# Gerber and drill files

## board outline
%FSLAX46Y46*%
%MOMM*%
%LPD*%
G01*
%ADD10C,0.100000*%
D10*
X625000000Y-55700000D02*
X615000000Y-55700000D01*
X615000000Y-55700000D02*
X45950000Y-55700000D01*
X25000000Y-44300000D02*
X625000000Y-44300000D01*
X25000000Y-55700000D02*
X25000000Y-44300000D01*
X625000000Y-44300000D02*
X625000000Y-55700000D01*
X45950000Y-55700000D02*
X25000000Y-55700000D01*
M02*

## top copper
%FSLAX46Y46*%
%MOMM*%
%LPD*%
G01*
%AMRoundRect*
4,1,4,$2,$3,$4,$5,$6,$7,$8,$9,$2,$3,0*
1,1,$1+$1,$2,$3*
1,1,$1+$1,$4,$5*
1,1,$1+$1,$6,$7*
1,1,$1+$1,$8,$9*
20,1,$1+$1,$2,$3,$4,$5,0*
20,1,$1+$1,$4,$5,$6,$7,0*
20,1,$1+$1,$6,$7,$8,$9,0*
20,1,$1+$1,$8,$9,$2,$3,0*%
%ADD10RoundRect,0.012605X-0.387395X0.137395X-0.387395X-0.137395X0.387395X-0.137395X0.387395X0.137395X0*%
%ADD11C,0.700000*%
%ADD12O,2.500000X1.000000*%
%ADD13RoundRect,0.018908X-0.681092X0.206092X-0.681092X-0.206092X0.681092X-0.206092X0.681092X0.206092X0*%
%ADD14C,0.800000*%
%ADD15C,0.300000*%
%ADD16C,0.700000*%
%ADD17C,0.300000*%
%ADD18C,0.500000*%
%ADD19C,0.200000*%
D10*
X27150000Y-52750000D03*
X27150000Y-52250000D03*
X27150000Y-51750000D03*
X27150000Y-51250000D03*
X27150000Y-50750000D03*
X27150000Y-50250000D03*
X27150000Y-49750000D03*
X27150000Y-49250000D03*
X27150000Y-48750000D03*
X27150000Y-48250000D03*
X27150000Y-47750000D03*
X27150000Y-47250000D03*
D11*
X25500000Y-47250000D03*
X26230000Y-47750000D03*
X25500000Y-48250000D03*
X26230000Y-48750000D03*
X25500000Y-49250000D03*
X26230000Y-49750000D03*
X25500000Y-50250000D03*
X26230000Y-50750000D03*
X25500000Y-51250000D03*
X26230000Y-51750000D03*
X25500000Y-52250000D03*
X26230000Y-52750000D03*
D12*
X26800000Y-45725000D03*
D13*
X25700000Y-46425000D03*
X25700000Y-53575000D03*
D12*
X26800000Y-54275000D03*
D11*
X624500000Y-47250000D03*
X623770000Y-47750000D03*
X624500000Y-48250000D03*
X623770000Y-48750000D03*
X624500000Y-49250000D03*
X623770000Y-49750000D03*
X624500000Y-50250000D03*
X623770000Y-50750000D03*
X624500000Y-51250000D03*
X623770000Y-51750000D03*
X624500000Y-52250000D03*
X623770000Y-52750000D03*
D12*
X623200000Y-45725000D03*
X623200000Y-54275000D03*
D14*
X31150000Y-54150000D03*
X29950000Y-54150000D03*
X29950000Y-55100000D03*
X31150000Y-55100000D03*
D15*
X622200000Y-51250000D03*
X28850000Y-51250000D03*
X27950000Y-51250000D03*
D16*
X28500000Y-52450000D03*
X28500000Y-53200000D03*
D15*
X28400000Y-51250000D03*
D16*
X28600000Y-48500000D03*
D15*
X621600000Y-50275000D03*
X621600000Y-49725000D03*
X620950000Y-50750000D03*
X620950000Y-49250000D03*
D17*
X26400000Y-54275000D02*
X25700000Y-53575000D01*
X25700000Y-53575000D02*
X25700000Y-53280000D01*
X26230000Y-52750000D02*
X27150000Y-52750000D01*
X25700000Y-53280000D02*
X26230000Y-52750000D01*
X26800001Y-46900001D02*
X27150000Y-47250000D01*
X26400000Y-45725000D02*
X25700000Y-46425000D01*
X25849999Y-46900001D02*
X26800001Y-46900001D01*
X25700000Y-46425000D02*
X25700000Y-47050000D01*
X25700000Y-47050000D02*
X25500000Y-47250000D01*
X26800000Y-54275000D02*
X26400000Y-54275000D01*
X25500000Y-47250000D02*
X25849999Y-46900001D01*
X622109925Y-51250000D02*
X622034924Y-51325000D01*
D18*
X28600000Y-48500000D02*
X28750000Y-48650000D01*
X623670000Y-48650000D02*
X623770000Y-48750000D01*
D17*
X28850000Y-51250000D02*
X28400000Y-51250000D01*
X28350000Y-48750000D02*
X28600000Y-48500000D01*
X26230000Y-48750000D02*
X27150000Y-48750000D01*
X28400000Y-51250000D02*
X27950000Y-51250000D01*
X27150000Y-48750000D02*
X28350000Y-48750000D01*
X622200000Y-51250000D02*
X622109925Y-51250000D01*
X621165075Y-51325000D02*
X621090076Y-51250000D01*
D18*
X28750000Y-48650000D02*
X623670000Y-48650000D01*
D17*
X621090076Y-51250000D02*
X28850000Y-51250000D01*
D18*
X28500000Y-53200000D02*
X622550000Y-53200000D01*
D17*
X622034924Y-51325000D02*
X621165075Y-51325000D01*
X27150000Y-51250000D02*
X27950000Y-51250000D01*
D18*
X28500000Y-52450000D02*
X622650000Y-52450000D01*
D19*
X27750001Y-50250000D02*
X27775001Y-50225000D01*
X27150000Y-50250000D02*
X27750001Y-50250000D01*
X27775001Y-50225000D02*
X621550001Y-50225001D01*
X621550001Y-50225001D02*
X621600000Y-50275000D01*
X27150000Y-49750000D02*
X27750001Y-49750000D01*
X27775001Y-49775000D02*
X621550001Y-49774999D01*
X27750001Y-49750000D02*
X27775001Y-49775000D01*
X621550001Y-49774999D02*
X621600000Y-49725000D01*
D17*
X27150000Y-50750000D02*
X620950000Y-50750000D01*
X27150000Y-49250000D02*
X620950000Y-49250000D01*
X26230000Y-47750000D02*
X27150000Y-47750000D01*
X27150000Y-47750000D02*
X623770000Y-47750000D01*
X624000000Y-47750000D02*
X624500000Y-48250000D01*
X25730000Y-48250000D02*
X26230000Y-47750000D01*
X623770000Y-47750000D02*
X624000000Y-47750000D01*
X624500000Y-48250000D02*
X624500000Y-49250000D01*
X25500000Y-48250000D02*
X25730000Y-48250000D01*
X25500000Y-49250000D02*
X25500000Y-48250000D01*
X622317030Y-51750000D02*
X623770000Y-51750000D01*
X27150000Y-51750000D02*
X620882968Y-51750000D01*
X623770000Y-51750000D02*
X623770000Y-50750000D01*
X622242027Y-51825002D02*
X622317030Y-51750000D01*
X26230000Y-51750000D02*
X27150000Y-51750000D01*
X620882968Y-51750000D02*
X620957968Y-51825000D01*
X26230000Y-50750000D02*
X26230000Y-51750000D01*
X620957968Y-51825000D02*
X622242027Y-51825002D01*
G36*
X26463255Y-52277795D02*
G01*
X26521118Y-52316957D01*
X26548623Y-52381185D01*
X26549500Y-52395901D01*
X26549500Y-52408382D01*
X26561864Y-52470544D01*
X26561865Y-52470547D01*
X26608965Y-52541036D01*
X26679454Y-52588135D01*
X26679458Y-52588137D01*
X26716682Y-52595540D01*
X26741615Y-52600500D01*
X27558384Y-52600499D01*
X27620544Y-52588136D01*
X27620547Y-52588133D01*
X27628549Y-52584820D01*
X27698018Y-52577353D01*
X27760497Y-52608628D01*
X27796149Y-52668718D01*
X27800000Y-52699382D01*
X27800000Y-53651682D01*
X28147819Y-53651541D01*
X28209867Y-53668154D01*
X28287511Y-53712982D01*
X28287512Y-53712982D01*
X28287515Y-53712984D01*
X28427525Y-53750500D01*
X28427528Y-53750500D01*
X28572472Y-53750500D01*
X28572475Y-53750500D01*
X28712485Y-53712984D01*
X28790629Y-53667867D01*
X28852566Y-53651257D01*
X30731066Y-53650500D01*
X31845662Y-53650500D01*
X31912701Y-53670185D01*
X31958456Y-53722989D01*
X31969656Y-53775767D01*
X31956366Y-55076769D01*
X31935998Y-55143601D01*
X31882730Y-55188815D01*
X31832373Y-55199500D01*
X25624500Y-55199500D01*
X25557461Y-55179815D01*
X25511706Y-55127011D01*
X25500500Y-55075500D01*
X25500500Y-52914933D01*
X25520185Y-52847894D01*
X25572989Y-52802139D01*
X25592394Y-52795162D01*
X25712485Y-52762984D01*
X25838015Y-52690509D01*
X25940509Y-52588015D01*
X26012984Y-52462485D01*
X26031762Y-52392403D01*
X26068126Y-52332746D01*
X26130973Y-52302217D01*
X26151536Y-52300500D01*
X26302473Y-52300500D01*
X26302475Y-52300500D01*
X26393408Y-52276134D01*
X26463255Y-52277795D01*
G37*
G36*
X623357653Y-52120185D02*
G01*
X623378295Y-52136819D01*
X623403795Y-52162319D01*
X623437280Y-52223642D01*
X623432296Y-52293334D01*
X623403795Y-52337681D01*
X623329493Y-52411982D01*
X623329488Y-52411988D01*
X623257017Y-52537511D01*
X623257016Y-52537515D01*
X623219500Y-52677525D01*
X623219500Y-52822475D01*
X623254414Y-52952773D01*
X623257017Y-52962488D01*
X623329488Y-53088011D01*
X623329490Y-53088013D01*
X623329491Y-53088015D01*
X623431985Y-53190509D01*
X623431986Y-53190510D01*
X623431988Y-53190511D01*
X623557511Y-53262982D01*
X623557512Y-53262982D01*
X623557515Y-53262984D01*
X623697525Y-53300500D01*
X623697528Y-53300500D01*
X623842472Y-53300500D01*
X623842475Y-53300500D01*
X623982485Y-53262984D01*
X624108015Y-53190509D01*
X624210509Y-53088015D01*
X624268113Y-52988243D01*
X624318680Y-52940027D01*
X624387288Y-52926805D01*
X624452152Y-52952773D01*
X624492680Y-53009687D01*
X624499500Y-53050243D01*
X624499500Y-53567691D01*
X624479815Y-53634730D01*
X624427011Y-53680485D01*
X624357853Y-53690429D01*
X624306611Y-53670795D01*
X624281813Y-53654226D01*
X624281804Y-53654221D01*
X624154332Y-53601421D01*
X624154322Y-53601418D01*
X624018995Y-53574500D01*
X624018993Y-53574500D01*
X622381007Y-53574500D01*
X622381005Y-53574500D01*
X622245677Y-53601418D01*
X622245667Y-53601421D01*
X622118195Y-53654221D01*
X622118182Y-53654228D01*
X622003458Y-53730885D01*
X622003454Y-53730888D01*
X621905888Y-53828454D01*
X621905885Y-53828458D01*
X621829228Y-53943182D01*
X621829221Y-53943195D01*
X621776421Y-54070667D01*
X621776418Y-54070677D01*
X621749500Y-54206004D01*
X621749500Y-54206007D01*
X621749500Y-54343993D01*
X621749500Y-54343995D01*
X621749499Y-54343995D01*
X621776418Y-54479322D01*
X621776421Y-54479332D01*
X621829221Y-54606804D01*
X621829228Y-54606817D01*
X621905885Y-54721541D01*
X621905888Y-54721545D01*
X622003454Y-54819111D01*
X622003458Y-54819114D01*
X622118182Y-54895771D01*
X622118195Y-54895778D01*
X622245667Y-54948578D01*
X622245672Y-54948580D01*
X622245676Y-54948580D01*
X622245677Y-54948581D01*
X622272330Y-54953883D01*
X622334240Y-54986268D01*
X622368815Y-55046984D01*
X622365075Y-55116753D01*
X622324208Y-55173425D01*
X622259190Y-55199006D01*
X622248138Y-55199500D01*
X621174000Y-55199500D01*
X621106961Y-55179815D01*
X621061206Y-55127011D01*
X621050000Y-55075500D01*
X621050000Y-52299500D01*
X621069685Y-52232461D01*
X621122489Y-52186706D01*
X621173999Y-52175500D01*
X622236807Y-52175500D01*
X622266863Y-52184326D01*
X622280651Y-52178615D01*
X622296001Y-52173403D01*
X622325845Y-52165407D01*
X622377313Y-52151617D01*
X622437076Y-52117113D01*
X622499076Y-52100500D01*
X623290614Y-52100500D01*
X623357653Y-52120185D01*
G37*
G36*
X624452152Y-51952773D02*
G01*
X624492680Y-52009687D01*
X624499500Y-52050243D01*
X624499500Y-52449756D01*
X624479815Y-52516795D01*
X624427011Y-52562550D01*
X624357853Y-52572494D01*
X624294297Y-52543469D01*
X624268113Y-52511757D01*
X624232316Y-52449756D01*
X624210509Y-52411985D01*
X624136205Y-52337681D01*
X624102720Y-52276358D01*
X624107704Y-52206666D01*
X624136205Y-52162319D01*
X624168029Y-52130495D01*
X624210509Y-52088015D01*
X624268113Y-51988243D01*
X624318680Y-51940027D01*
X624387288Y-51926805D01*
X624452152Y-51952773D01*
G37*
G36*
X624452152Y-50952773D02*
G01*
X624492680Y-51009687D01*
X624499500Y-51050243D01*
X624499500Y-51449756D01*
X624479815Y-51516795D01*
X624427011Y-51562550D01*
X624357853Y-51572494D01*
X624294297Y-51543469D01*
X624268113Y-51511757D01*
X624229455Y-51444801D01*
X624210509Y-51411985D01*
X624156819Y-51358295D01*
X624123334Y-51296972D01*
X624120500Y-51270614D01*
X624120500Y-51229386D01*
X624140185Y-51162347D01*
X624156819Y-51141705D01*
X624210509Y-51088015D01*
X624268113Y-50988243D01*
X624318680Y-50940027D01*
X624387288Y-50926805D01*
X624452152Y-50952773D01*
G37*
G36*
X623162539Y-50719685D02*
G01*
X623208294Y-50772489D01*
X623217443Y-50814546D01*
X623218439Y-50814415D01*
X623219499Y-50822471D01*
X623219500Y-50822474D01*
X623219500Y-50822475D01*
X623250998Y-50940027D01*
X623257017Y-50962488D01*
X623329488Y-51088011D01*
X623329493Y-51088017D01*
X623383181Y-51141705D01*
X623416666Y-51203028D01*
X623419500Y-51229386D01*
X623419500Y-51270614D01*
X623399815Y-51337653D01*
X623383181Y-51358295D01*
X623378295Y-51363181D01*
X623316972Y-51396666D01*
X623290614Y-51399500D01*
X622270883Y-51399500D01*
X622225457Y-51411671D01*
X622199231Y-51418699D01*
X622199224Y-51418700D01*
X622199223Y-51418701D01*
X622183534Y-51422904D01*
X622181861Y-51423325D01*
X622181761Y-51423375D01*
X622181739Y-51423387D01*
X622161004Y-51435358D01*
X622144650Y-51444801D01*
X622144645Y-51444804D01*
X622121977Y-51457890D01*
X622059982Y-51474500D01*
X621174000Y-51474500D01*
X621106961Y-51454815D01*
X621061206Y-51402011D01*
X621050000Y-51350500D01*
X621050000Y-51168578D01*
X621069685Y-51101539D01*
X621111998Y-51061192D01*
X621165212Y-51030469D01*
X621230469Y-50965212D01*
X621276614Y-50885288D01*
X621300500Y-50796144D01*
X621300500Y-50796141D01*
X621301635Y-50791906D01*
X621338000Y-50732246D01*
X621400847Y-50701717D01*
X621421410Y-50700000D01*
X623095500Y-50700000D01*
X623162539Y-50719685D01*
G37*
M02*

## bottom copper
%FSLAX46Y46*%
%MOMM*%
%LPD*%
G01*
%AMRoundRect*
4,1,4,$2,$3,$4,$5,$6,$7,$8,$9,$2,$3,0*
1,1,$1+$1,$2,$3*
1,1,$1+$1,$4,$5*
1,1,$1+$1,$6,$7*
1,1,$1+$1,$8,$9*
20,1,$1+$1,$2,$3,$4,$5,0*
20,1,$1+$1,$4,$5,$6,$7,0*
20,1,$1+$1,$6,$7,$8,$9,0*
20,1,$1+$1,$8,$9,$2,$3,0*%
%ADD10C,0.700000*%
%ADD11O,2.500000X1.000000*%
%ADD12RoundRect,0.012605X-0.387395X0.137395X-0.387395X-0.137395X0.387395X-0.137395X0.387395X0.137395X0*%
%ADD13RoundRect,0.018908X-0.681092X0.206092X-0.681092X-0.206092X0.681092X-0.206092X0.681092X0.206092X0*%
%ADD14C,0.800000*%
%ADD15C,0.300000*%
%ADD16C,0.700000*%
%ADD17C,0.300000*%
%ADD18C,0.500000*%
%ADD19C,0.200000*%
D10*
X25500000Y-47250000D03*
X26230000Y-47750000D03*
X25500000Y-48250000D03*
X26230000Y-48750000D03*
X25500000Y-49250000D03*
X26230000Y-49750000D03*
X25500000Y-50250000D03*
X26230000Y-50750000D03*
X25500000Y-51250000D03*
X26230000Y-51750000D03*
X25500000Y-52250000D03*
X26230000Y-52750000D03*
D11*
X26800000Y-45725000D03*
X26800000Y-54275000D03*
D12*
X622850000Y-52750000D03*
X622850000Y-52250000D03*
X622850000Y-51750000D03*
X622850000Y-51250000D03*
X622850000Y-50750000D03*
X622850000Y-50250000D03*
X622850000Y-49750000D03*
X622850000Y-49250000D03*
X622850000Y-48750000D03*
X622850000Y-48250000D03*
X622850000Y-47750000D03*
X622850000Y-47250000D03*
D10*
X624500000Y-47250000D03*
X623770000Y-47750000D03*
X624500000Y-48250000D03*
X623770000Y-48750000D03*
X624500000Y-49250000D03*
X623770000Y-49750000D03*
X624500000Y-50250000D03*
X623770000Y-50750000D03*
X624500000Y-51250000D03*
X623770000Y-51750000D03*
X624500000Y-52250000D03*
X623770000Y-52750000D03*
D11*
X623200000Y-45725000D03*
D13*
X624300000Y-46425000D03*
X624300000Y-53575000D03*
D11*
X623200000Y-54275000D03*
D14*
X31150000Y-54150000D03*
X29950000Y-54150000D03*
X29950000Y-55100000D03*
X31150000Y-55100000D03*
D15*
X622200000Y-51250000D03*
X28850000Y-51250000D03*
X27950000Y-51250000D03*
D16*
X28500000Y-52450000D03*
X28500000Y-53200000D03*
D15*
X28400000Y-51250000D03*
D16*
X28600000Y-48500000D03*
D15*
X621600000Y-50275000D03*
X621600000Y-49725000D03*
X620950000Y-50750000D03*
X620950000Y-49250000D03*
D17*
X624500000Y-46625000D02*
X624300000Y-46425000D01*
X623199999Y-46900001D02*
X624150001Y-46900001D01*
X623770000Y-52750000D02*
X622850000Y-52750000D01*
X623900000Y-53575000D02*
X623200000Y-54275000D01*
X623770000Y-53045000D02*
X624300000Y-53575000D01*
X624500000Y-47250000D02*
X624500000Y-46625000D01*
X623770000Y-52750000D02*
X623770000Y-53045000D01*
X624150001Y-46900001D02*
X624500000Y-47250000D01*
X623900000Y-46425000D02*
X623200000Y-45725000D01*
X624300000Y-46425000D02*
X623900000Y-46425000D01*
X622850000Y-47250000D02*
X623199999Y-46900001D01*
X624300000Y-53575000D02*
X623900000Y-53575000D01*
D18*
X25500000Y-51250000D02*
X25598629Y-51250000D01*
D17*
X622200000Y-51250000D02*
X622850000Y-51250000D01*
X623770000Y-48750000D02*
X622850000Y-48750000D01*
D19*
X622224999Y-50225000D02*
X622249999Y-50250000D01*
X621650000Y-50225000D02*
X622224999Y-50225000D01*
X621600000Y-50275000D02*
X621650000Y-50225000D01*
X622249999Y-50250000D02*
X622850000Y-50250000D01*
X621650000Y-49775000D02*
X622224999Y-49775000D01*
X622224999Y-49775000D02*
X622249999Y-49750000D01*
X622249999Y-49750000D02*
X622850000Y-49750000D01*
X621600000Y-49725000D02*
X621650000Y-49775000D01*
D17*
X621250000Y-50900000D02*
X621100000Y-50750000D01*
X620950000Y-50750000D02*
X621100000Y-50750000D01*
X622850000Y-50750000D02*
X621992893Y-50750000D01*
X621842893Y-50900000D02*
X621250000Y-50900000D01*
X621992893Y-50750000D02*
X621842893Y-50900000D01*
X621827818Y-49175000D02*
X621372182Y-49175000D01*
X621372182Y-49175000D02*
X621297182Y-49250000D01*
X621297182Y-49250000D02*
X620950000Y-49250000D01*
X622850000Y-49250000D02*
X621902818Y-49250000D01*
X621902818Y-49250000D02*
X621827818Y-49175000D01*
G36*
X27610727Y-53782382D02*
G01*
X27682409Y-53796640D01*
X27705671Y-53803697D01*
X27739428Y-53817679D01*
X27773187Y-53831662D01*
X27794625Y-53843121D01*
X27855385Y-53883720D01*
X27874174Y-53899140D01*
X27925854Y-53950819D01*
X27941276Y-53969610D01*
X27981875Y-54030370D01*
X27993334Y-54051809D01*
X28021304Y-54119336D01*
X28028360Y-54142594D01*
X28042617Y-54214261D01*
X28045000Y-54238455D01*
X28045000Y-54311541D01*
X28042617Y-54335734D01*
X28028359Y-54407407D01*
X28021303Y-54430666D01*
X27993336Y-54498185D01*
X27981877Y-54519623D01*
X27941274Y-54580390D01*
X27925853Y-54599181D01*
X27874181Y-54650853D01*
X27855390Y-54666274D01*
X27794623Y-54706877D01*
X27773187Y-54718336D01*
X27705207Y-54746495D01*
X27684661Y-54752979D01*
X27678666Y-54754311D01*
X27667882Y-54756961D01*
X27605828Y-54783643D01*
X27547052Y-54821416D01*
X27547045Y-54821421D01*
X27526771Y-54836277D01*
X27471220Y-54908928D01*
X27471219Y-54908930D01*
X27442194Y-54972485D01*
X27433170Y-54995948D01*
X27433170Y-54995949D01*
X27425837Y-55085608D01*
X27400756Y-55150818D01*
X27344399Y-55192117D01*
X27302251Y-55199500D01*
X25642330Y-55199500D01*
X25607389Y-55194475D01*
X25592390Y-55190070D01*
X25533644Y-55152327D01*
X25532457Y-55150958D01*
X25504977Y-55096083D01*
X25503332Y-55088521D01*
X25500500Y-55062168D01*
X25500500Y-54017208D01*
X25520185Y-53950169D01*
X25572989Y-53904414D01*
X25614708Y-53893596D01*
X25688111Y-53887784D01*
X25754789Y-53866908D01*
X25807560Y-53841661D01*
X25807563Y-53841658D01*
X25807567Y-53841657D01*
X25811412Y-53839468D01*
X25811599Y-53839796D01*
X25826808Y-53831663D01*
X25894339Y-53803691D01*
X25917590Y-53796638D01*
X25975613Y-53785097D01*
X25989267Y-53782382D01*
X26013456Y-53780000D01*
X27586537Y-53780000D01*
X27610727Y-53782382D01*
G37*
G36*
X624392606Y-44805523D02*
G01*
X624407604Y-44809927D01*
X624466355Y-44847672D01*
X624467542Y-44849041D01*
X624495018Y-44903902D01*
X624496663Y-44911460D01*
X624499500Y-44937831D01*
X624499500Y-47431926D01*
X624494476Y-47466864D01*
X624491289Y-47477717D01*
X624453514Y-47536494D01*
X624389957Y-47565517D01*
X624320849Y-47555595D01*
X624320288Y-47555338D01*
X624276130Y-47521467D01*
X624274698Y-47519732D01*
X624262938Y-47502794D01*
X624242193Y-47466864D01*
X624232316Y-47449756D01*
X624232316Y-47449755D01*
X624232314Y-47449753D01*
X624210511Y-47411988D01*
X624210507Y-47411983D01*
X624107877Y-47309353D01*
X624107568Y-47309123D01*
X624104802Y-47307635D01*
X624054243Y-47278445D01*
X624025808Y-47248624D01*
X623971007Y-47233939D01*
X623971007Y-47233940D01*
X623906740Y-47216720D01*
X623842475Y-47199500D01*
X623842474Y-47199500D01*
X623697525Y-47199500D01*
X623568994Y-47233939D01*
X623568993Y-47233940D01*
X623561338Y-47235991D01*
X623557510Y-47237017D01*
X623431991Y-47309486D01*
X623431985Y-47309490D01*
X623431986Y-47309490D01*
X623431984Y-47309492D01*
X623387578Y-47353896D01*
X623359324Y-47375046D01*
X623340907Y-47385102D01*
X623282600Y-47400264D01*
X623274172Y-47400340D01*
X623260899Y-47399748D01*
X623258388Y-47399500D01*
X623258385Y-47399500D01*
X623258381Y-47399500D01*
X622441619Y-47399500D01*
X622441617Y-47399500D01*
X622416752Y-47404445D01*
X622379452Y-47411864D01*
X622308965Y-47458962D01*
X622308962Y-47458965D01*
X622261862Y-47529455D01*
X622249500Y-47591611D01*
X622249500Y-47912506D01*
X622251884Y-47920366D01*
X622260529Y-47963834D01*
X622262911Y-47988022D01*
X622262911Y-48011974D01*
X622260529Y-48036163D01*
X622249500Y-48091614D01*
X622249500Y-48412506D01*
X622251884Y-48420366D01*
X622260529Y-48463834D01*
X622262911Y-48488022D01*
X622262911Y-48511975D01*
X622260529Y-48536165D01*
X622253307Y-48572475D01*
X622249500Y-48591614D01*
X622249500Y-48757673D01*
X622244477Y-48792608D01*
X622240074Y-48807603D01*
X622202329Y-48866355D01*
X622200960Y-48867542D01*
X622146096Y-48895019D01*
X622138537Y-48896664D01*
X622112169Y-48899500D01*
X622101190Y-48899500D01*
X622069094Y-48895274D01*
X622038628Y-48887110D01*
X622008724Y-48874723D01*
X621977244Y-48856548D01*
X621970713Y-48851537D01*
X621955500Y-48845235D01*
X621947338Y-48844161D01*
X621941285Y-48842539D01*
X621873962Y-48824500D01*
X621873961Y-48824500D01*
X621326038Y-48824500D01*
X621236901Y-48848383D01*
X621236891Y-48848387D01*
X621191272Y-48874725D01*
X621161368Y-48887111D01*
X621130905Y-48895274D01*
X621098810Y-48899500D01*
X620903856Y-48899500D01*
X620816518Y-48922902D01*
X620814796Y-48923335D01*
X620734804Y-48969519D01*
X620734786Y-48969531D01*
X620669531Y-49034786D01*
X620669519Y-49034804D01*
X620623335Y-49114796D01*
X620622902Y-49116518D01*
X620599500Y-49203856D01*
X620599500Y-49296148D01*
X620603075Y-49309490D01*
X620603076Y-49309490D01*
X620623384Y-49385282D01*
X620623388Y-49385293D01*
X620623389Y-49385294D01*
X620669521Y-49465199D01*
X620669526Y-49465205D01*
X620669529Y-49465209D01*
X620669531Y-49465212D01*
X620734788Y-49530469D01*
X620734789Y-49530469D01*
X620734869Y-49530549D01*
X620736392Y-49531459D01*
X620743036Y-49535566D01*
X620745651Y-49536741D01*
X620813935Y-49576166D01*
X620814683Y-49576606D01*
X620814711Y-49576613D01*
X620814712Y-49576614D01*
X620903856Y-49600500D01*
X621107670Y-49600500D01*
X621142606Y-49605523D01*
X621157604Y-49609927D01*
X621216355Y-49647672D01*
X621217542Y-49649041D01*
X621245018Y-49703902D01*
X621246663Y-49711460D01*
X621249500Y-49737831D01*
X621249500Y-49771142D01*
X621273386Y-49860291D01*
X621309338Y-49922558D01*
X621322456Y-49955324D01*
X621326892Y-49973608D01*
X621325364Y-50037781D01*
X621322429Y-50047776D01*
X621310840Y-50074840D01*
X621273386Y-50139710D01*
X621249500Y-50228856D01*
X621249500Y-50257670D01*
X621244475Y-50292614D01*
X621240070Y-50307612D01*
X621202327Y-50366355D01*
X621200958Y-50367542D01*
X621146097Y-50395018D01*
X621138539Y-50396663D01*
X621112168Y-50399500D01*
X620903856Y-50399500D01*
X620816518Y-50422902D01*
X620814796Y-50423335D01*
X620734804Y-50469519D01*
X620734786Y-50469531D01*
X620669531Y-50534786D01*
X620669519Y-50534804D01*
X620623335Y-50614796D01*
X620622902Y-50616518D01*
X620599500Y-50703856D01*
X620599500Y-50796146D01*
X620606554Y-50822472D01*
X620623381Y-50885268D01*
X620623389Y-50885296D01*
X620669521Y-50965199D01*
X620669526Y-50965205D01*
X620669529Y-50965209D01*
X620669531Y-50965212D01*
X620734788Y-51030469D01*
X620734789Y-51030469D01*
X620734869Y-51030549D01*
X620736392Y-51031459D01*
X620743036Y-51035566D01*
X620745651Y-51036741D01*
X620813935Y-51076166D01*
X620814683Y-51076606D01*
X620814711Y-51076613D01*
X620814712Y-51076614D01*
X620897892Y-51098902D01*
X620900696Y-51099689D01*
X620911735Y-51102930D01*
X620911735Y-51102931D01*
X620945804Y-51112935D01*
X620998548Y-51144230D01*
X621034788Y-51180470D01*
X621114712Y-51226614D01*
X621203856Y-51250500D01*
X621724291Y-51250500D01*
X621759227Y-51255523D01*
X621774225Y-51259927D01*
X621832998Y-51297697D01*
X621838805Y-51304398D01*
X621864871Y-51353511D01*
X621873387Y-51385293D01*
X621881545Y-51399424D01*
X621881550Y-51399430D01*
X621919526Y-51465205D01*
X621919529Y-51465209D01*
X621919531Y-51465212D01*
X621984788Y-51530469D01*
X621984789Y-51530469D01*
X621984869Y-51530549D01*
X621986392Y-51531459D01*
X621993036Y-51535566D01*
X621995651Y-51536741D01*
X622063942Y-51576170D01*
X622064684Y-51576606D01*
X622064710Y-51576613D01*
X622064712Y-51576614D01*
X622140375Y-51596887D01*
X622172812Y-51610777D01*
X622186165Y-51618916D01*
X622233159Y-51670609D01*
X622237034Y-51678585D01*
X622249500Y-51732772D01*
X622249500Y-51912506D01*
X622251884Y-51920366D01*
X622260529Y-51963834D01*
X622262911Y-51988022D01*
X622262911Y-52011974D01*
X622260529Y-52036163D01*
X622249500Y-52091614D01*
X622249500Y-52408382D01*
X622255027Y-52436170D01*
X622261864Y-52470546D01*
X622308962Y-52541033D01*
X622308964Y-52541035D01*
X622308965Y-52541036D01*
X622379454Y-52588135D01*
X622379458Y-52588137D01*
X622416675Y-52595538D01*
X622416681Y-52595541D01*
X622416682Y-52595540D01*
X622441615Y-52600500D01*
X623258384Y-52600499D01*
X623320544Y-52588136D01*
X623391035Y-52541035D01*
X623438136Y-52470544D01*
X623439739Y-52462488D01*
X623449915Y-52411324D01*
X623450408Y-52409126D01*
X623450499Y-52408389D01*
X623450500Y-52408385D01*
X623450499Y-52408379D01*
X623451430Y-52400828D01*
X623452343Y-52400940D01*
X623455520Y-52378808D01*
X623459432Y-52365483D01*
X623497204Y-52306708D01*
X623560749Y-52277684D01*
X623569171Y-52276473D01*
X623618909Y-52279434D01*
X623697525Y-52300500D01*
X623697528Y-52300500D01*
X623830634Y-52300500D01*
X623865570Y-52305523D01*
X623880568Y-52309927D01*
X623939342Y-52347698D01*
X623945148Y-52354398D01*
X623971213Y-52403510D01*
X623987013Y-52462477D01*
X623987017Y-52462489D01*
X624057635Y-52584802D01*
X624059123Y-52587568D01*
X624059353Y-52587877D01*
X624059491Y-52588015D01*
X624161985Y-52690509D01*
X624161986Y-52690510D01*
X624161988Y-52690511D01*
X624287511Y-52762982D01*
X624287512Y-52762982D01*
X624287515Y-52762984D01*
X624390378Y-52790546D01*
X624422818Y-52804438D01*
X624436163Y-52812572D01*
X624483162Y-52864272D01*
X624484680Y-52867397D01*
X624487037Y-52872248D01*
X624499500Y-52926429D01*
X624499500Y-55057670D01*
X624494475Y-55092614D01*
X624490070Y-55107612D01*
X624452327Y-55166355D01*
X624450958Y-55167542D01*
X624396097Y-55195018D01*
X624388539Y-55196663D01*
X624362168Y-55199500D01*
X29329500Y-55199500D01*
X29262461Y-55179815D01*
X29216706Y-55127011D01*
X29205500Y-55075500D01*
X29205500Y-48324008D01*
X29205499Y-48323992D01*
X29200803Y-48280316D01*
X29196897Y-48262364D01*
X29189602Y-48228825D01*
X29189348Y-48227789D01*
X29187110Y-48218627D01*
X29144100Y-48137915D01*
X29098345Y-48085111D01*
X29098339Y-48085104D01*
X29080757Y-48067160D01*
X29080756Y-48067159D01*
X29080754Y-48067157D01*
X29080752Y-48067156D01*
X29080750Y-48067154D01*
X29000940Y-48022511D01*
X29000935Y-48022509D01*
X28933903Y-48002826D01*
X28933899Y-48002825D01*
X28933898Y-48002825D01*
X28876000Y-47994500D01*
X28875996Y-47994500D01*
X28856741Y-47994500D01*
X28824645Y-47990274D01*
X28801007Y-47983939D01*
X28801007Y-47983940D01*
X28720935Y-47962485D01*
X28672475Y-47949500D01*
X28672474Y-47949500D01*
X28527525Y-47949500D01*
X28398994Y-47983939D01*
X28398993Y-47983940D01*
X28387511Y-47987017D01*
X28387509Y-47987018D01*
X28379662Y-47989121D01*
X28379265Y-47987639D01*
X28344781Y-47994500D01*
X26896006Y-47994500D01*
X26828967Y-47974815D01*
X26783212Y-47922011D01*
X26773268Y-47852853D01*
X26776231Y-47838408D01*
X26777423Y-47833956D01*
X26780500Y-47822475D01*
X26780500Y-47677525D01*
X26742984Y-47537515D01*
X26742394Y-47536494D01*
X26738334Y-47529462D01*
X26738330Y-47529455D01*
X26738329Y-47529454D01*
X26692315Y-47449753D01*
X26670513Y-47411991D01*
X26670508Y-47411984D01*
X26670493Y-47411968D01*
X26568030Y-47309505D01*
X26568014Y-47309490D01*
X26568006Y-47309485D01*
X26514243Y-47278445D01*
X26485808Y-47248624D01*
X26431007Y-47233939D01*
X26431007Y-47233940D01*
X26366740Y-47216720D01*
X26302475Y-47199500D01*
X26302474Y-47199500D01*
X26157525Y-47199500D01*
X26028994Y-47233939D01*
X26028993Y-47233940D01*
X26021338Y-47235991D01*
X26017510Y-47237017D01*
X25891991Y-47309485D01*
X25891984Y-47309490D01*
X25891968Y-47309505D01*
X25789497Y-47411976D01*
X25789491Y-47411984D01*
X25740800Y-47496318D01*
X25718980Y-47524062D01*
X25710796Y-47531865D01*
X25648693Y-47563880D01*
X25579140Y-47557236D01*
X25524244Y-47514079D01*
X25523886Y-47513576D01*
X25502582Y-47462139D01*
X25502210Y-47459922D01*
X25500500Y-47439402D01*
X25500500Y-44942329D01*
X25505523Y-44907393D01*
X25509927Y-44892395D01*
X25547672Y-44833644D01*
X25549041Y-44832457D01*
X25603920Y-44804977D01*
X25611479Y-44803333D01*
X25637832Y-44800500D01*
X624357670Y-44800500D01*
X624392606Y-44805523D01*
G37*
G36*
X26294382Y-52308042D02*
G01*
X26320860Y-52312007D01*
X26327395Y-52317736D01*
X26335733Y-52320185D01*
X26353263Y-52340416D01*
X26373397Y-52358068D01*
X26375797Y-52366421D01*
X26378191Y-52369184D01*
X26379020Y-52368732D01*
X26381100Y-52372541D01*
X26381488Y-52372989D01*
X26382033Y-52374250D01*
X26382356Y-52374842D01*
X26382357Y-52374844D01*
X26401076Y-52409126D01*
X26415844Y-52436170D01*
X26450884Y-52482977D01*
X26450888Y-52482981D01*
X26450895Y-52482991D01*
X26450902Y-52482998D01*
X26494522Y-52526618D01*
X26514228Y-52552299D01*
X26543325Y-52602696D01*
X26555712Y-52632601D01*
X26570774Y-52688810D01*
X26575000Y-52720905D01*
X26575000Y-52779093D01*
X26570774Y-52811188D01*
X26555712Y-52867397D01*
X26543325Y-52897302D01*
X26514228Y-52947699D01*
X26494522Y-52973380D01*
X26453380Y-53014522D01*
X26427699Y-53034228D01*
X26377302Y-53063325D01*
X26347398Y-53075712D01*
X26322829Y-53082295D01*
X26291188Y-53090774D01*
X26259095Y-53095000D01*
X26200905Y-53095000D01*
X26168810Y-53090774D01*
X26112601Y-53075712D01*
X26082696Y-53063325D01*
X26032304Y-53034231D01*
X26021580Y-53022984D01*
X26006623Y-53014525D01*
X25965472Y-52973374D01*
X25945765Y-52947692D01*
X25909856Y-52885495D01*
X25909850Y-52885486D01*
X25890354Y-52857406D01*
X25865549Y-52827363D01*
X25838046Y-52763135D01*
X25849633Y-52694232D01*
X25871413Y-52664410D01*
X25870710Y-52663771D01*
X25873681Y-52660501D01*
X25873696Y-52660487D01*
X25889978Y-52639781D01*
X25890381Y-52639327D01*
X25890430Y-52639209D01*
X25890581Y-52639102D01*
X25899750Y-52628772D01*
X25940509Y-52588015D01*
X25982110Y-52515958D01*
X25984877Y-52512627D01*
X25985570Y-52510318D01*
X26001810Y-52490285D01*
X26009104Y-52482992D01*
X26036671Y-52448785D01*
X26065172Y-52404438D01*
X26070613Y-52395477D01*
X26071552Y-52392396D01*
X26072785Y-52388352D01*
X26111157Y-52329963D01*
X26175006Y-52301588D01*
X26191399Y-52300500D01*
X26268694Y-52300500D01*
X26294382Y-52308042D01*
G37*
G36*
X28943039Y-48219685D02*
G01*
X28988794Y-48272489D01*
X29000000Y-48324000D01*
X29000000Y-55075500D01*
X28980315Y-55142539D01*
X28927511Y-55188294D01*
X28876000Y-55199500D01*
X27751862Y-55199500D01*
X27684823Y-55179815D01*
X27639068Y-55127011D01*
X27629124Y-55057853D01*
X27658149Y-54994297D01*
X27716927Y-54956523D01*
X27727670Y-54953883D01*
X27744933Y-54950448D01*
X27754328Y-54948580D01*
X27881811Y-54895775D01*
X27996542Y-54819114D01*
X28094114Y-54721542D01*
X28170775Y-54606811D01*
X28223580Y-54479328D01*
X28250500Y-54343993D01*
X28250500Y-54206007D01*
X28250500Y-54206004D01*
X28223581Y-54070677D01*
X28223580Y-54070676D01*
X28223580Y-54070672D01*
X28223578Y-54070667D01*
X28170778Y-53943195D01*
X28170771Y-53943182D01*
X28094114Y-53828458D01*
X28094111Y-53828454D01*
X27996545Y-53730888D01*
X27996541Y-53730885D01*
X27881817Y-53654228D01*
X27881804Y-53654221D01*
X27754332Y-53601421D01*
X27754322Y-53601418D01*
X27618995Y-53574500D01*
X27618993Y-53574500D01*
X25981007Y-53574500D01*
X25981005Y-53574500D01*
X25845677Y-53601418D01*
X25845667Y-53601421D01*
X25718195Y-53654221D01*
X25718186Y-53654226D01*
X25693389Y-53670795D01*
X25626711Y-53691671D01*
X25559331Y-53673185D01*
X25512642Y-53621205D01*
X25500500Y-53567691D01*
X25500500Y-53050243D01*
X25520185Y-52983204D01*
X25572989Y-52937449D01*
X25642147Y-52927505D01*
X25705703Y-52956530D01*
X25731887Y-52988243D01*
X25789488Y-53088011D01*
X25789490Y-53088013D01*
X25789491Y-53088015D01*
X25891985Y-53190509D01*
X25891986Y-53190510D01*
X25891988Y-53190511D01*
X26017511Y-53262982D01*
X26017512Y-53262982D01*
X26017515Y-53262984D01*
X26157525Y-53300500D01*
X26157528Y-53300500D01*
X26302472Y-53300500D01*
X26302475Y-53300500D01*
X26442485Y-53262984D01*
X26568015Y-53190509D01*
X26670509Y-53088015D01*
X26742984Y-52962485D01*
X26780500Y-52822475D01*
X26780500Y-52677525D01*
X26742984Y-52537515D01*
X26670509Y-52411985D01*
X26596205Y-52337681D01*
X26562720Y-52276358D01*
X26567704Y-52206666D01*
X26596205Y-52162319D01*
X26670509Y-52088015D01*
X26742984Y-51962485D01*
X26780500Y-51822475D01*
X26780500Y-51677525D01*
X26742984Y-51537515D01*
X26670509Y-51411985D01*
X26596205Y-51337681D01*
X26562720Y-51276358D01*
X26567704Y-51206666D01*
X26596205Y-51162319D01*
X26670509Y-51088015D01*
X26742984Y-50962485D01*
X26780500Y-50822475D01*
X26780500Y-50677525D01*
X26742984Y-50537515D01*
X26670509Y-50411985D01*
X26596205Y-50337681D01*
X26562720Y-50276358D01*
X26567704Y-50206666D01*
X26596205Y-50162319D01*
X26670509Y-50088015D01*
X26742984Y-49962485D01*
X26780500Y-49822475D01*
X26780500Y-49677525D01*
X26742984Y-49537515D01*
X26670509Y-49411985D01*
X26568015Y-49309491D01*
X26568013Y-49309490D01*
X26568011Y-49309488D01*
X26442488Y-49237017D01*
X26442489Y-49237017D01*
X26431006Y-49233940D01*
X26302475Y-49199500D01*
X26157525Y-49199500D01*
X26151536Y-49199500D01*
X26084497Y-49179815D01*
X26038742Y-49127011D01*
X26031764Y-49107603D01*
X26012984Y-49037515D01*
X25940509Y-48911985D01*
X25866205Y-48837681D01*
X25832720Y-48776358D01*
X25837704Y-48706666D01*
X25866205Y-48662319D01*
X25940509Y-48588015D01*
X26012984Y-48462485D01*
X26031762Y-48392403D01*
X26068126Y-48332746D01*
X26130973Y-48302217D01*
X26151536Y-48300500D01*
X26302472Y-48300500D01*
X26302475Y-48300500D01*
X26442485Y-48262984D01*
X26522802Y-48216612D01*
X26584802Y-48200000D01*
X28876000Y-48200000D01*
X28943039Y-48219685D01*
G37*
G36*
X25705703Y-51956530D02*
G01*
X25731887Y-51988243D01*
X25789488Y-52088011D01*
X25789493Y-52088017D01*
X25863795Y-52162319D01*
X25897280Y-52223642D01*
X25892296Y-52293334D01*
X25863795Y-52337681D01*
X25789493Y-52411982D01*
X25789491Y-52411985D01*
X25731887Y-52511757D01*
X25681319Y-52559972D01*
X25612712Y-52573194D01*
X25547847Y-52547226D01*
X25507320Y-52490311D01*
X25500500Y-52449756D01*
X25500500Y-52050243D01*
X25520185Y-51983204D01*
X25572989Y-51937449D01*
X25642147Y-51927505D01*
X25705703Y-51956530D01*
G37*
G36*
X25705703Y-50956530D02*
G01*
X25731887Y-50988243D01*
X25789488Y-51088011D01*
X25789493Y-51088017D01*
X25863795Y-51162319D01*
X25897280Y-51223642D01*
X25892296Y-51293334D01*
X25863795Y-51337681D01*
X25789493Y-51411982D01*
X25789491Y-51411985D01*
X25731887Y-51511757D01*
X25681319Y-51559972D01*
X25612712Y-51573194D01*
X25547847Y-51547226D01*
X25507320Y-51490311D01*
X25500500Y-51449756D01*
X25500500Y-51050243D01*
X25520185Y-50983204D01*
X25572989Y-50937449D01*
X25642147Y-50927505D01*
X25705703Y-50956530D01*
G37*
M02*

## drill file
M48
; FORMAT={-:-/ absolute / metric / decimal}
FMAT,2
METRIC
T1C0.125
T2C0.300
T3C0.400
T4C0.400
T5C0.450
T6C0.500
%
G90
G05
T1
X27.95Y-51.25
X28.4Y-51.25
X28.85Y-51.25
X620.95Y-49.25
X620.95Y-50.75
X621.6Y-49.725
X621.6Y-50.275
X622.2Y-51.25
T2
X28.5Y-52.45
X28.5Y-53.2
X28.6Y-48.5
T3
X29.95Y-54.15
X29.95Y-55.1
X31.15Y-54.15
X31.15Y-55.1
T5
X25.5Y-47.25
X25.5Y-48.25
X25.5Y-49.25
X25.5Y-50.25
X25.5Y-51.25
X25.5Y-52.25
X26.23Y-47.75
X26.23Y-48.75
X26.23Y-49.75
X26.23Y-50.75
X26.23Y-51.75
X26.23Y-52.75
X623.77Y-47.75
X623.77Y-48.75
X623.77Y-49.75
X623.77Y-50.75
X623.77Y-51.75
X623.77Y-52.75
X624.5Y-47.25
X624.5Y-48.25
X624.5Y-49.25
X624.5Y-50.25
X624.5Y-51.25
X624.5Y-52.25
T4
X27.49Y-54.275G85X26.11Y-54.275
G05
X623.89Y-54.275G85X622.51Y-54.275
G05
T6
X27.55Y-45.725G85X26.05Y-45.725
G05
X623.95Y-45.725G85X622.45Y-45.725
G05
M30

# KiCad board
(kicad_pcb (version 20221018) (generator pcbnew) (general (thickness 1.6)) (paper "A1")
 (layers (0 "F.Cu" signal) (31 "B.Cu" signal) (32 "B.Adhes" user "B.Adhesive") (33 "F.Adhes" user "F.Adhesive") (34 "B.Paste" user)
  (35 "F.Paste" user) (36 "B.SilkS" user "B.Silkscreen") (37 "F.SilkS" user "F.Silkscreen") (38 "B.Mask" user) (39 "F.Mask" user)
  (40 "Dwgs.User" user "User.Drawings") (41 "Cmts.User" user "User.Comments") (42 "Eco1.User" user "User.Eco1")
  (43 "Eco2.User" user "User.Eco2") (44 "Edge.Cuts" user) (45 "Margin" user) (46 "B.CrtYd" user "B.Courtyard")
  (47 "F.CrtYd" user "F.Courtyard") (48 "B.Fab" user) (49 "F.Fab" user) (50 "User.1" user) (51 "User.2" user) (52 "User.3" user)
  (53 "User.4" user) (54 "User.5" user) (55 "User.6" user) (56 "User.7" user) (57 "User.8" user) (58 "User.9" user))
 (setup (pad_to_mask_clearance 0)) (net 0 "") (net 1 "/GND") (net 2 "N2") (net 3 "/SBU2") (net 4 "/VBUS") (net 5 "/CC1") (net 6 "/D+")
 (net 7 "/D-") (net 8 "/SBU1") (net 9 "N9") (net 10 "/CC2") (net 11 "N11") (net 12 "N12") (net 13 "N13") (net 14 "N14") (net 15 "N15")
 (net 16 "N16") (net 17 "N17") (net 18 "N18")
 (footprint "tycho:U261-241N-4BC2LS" (layer "F.Cu") (at 25 50 -90)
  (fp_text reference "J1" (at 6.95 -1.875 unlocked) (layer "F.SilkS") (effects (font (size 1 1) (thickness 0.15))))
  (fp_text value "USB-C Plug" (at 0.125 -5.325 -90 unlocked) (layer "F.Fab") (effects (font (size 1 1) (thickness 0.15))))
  (pad "A1" smd roundrect (at 2.75 -2.15 270) (size 0.3 0.8) (layers "F.Cu" "F.Paste" "F.Mask") (roundrect_rratio 0.04201680672)
   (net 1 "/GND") (thermal_bridge_angle 45))
  (pad "A2" smd roundrect (at 2.25 -2.15 270) (size 0.3 0.8) (layers "F.Cu" "F.Paste" "F.Mask") (roundrect_rratio 0.04201680672)
   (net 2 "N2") (thermal_bridge_angle 45))
  (pad "A3" smd roundrect (at 1.75 -2.15 270) (size 0.3 0.8) (layers "F.Cu" "F.Paste" "F.Mask") (roundrect_rratio 0.04201680672)
   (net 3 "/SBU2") (thermal_bridge_angle 45))
  (pad "A4" smd roundrect (at 1.25 -2.15 270) (size 0.3 0.8) (layers "F.Cu" "F.Paste" "F.Mask") (roundrect_rratio 0.04201680672)
   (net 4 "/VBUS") (thermal_bridge_angle 45))
  (pad "A5" smd roundrect (at 0.75 -2.15 270) (size 0.3 0.8) (layers "F.Cu" "F.Paste" "F.Mask") (roundrect_rratio 0.04201680672)
   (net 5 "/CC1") (thermal_bridge_angle 45))
  (pad "A6" smd roundrect (at 0.25 -2.15 270) (size 0.3 0.8) (layers "F.Cu" "F.Paste" "F.Mask") (roundrect_rratio 0.04201680672)
   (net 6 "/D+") (thermal_bridge_angle 45))
  (pad "A7" smd roundrect (at -0.25 -2.15 270) (size 0.3 0.8) (layers "F.Cu" "F.Paste" "F.Mask") (roundrect_rratio 0.04201680672)
   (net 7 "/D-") (thermal_bridge_angle 45))
  (pad "A8" smd roundrect (at -0.75 -2.15 270) (size 0.3 0.8) (layers "F.Cu" "F.Paste" "F.Mask") (roundrect_rratio 0.04201680672)
   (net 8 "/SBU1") (thermal_bridge_angle 45))
  (pad "A9" smd roundrect (at -1.25 -2.15 270) (size 0.3 0.8) (layers "F.Cu" "F.Paste" "F.Mask") (roundrect_rratio 0.04201680672)
   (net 4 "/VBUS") (thermal_bridge_angle 45))
  (pad "A10" smd roundrect (at -1.75 -2.15 270) (size 0.3 0.8) (layers "F.Cu" "F.Paste" "F.Mask") (roundrect_rratio 0.04201680672)
   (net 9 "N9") (thermal_bridge_angle 45))
  (pad "A11" smd roundrect (at -2.25 -2.15 270) (size 0.3 0.8) (layers "F.Cu" "F.Paste" "F.Mask") (roundrect_rratio 0.04201680672)
   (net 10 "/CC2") (thermal_bridge_angle 45))
  (pad "A12" smd roundrect (at -2.75 -2.15 270) (size 0.3 0.8) (layers "F.Cu" "F.Paste" "F.Mask") (roundrect_rratio 0.04201680672)
   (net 1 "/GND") (thermal_bridge_angle 45))
  (pad "B1" thru_hole circle (at -2.75 -0.5 270) (size 0.7 0.7) (drill 0.45) (layers "*.Cu" "*.Mask") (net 1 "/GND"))
  (pad "B2" thru_hole circle (at -2.25 -1.23 270) (size 0.7 0.7) (drill 0.45) (layers "*.Cu" "*.Mask") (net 10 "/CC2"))
  (pad "B3" thru_hole circle (at -1.75 -0.5 270) (size 0.7 0.7) (drill 0.45) (layers "*.Cu" "*.Mask") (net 10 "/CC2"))
  (pad "B4" thru_hole circle (at -1.25 -1.23 270) (size 0.7 0.7) (drill 0.45) (layers "*.Cu" "*.Mask") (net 4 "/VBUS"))
  (pad "B5" thru_hole circle (at -0.75 -0.5 270) (size 0.7 0.7) (drill 0.45) (layers "*.Cu" "*.Mask") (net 10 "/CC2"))
  (pad "B6" thru_hole circle (at -0.25 -1.23 270) (size 0.7 0.7) (drill 0.45) (layers "*.Cu" "*.Mask") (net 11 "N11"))
  (pad "B7" thru_hole circle (at 0.25 -0.5 270) (size 0.7 0.7) (drill 0.45) (layers "*.Cu" "*.Mask") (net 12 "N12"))
  (pad "B8" thru_hole circle (at 0.75 -1.23 270) (size 0.7 0.7) (drill 0.45) (layers "*.Cu" "*.Mask") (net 3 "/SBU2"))
  (pad "B9" thru_hole circle (at 1.25 -0.5 270) (size 0.7 0.7) (drill 0.45) (layers "*.Cu" "*.Mask") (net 4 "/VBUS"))
  (pad "B10" thru_hole circle (at 1.75 -1.23 270) (size 0.7 0.7) (drill 0.45) (layers "*.Cu" "*.Mask") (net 3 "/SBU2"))
  (pad "B11" thru_hole circle (at 2.25 -0.5 270) (size 0.7 0.7) (drill 0.45) (layers "*.Cu" "*.Mask") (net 4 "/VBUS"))
  (pad "B12" thru_hole circle (at 2.75 -1.23 270) (size 0.7 0.7) (drill 0.45) (layers "*.Cu" "*.Mask") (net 1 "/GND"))
  (pad "GND" thru_hole oval (at -4.275 -1.8 270) (size 1 2.5) (drill oval 0.5 2) (layers "*.Cu" "*.Mask") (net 1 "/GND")
   (thermal_bridge_angle 45))
  (pad "GND" smd roundrect (at -3.575 -0.7 270) (size 0.45 1.4) (layers "F.Cu" "F.Paste" "F.Mask") (roundrect_rratio 0.04201680672)
   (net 1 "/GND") (thermal_bridge_angle 45))
  (pad "GND" smd roundrect (at 3.575 -0.7 270) (size 0.45 1.4) (layers "F.Cu" "F.Paste" "F.Mask") (roundrect_rratio 0.04201680672)
   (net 1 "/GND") (thermal_bridge_angle 45))
  (pad "GND" thru_hole oval (at 4.275 -1.8 270) (size 1 2.5) (drill oval 0.4 1.78) (layers "*.Cu" "*.Mask") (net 1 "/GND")
   (thermal_bridge_angle 45)))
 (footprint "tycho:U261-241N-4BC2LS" (layer "B.Cu") (at 625 50 -90)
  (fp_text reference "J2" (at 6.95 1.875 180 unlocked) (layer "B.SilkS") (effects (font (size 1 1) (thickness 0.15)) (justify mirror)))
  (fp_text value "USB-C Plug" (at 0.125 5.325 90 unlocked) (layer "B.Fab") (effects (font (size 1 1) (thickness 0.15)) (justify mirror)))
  (pad "A1" smd roundrect (at 2.75 2.15 270) (size 0.3 0.8) (layers "B.Cu" "B.Paste" "B.Mask") (roundrect_rratio 0.04201680672)
   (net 1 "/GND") (thermal_bridge_angle 45))
  (pad "A2" smd roundrect (at 2.25 2.15 270) (size 0.3 0.8) (layers "B.Cu" "B.Paste" "B.Mask") (roundrect_rratio 0.04201680672)
   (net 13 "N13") (thermal_bridge_angle 45))
  (pad "A3" smd roundrect (at 1.75 2.15 270) (size 0.3 0.8) (layers "B.Cu" "B.Paste" "B.Mask") (roundrect_rratio 0.04201680672)
   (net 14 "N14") (thermal_bridge_angle 45))
  (pad "A4" smd roundrect (at 1.25 2.15 270) (size 0.3 0.8) (layers "B.Cu" "B.Paste" "B.Mask") (roundrect_rratio 0.04201680672)
   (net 4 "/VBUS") (thermal_bridge_angle 45))
  (pad "A5" smd roundrect (at 0.75 2.15 270) (size 0.3 0.8) (layers "B.Cu" "B.Paste" "B.Mask") (roundrect_rratio 0.04201680672)
   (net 5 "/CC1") (thermal_bridge_angle 45))
  (pad "A6" smd roundrect (at 0.25 2.15 270) (size 0.3 0.8) (layers "B.Cu" "B.Paste" "B.Mask") (roundrect_rratio 0.04201680672)
   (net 6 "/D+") (thermal_bridge_angle 45))
  (pad "A7" smd roundrect (at -0.25 2.15 270) (size 0.3 0.8) (layers "B.Cu" "B.Paste" "B.Mask") (roundrect_rratio 0.04201680672)
   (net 7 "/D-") (thermal_bridge_angle 45))
  (pad "A8" smd roundrect (at -0.75 2.15 270) (size 0.3 0.8) (layers "B.Cu" "B.Paste" "B.Mask") (roundrect_rratio 0.04201680672)
   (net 8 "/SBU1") (thermal_bridge_angle 45))
  (pad "A9" smd roundrect (at -1.25 2.15 270) (size 0.3 0.8) (layers "B.Cu" "B.Paste" "B.Mask") (roundrect_rratio 0.04201680672)
   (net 4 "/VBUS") (thermal_bridge_angle 45))
  (pad "A10" smd roundrect (at -1.75 2.15 270) (size 0.3 0.8) (layers "B.Cu" "B.Paste" "B.Mask") (roundrect_rratio 0.04201680672)
   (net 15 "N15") (thermal_bridge_angle 45))
  (pad "A11" smd roundrect (at -2.25 2.15 270) (size 0.3 0.8) (layers "B.Cu" "B.Paste" "B.Mask") (roundrect_rratio 0.04201680672)
   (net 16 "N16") (thermal_bridge_angle 45))
  (pad "A12" smd roundrect (at -2.75 2.15 270) (size 0.3 0.8) (layers "B.Cu" "B.Paste" "B.Mask") (roundrect_rratio 0.04201680672)
   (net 1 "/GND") (thermal_bridge_angle 45))
  (pad "B1" thru_hole circle (at -2.75 0.5 270) (size 0.7 0.7) (drill 0.45) (layers "*.Cu" "*.Mask") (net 1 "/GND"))
  (pad "B2" thru_hole circle (at -2.25 1.23 270) (size 0.7 0.7) (drill 0.45) (layers "*.Cu" "*.Mask") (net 10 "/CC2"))
  (pad "B3" thru_hole circle (at -1.75 0.5 270) (size 0.7 0.7) (drill 0.45) (layers "*.Cu" "*.Mask") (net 10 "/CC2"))
  (pad "B4" thru_hole circle (at -1.25 1.23 270) (size 0.7 0.7) (drill 0.45) (layers "*.Cu" "*.Mask") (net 4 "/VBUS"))
  (pad "B5" thru_hole circle (at -0.75 0.5 270) (size 0.7 0.7) (drill 0.45) (layers "*.Cu" "*.Mask") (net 10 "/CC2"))
  (pad "B6" thru_hole circle (at -0.25 1.23 270) (size 0.7 0.7) (drill 0.45) (layers "*.Cu" "*.Mask") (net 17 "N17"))
  (pad "B7" thru_hole circle (at 0.25 0.5 270) (size 0.7 0.7) (drill 0.45) (layers "*.Cu" "*.Mask") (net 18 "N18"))
  (pad "B8" thru_hole circle (at 0.75 1.23 270) (size 0.7 0.7) (drill 0.45) (layers "*.Cu" "*.Mask") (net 3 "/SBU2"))
  (pad "B9" thru_hole circle (at 1.25 0.5 270) (size 0.7 0.7) (drill 0.45) (layers "*.Cu" "*.Mask") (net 4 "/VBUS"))
  (pad "B10" thru_hole circle (at 1.75 1.23 270) (size 0.7 0.7) (drill 0.45) (layers "*.Cu" "*.Mask") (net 3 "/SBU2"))
  (pad "B11" thru_hole circle (at 2.25 0.5 270) (size 0.7 0.7) (drill 0.45) (layers "*.Cu" "*.Mask") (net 4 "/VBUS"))
  (pad "B12" thru_hole circle (at 2.75 1.23 270) (size 0.7 0.7) (drill 0.45) (layers "*.Cu" "*.Mask") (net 1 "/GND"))
  (pad "GND" thru_hole oval (at -4.275 1.8 270) (size 1 2.5) (drill oval 0.5 2) (layers "*.Cu" "*.Mask") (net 1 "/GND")
   (thermal_bridge_angle 45))
  (pad "GND" smd roundrect (at -3.575 0.7 270) (size 0.45 1.4) (layers "B.Cu" "B.Paste" "B.Mask") (roundrect_rratio 0.04201680672)
   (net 1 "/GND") (thermal_bridge_angle 45))
  (pad "GND" smd roundrect (at 3.575 0.7 270) (size 0.45 1.4) (layers "B.Cu" "B.Paste" "B.Mask") (roundrect_rratio 0.04201680672)
   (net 1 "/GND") (thermal_bridge_angle 45))
  (pad "GND" thru_hole oval (at 4.275 1.8 270) (size 1 2.5) (drill oval 0.4 1.78) (layers "*.Cu" "*.Mask") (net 1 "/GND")
   (thermal_bridge_angle 45)))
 (gr_line (start 625 55.7) (end 615 55.7) (stroke (width 0.1) (type default)) (layer "Edge.Cuts"))
 (gr_line (start 615 55.7) (end 45.95 55.7) (stroke (width 0.1) (type default)) (layer "Edge.Cuts"))
 (gr_line (start 25 44.3) (end 625 44.3) (stroke (width 0.1) (type default)) (layer "Edge.Cuts"))
 (gr_line (start 25 55.7) (end 25 44.3) (stroke (width 0.1) (type default)) (layer "Edge.Cuts"))
 (gr_line (start 625 44.3) (end 625 55.7) (stroke (width 0.1) (type default)) (layer "Edge.Cuts"))
 (gr_line (start 45.95 55.7) (end 25 55.7) (stroke (width 0.1) (type default)) (layer "Edge.Cuts"))
 (segment (start 26.4 54.275) (end 25.7 53.575) (width 0.3) (layer "F.Cu") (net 1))
 (segment (start 25.7 53.575) (end 25.7 53.28) (width 0.3) (layer "F.Cu") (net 1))
 (segment (start 26.23 52.75) (end 27.15 52.75) (width 0.3) (layer "F.Cu") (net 1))
 (segment (start 25.7 53.28) (end 26.23 52.75) (width 0.3) (layer "F.Cu") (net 1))
 (segment (start 26.800001 46.900001) (end 27.15 47.25) (width 0.3) (layer "F.Cu") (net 1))
 (segment (start 26.4 45.725) (end 25.7 46.425) (width 0.3) (layer "F.Cu") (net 1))
 (segment (start 25.849999 46.900001) (end 26.800001 46.900001) (width 0.3) (layer "F.Cu") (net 1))
 (segment (start 25.7 46.425) (end 25.7 47.05) (width 0.3) (layer "F.Cu") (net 1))
 (segment (start 25.7 47.05) (end 25.5 47.25) (width 0.3) (layer "F.Cu") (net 1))
 (segment (start 26.8 54.275) (end 26.4 54.275) (width 0.3) (layer "F.Cu") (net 1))
 (segment (start 25.5 47.25) (end 25.849999 46.900001) (width 0.3) (layer "F.Cu") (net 1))
 (via (at 31.15 54.15) (size 0.8) (drill 0.4) (layers "F.Cu" "B.Cu") (free) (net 1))
 (via (at 29.95 54.15) (size 0.8) (drill 0.4) (layers "F.Cu" "B.Cu") (free) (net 1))
 (via (at 29.95 55.1) (size 0.8) (drill 0.4) (layers "F.Cu" "B.Cu") (free) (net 1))
 (via (at 31.15 55.1) (size 0.8) (drill 0.4) (layers "F.Cu" "B.Cu") (free) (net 1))
 (segment (start 624.5 46.625) (end 624.3 46.425) (width 0.3) (layer "B.Cu") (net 1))
 (segment (start 623.199999 46.900001) (end 624.150001 46.900001) (width 0.3) (layer "B.Cu") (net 1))
 (segment (start 623.77 52.75) (end 622.85 52.75) (width 0.3) (layer "B.Cu") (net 1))
 (segment (start 623.9 53.575) (end 623.2 54.275) (width 0.3) (layer "B.Cu") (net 1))
 (segment (start 623.77 53.045) (end 624.3 53.575) (width 0.3) (layer "B.Cu") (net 1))
 (segment (start 624.5 47.25) (end 624.5 46.625) (width 0.3) (layer "B.Cu") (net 1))
 (segment (start 623.77 52.75) (end 623.77 53.045) (width 0.3) (layer "B.Cu") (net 1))
 (segment (start 624.150001 46.900001) (end 624.5 47.25) (width 0.3) (layer "B.Cu") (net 1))
 (segment (start 623.9 46.425) (end 623.2 45.725) (width 0.3) (layer "B.Cu") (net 1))
 (segment (start 624.3 46.425) (end 623.9 46.425) (width 0.3) (layer "B.Cu") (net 1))
 (segment (start 622.85 47.25) (end 623.199999 46.900001) (width 0.3) (layer "B.Cu") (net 1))
 (segment (start 624.3 53.575) (end 623.9 53.575) (width 0.3) (layer "B.Cu") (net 1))
 (segment (start 622.109925 51.25) (end 622.034924 51.325) (width 0.3) (layer "F.Cu") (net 4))
 (segment (start 28.6 48.5) (end 28.75 48.65) (width 0.5) (layer "F.Cu") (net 4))
 (segment (start 623.67 48.65) (end 623.77 48.75) (width 0.5) (layer "F.Cu") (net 4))
 (segment (start 28.85 51.25) (end 28.4 51.25) (width 0.3) (layer "F.Cu") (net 4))
 (segment (start 28.35 48.75) (end 28.6 48.5) (width 0.3) (layer "F.Cu") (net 4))
 (segment (start 26.23 48.75) (end 27.15 48.75) (width 0.3) (layer "F.Cu") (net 4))
 (segment (start 28.4 51.25) (end 27.95 51.25) (width 0.3) (layer "F.Cu") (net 4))
 (segment (start 27.15 48.75) (end 28.35 48.75) (width 0.3) (layer "F.Cu") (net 4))
 (segment (start 622.2 51.25) (end 622.109925 51.25) (width 0.3) (layer "F.Cu") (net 4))
 (segment (start 621.165075 51.325) (end 621.090076 51.25) (width 0.3) (layer "F.Cu") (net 4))
 (segment (start 28.75 48.65) (end 623.67 48.65) (width 0.5) (layer "F.Cu") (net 4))
 (segment (start 621.090076 51.25) (end 28.85 51.25) (width 0.3) (layer "F.Cu") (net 4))
 (segment (start 28.5 53.2) (end 622.55 53.2) (width 0.5) (layer "F.Cu") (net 4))
 (segment (start 622.034924 51.325) (end 621.165075 51.325) (width 0.3) (layer "F.Cu") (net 4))
 (segment (start 27.15 51.25) (end 27.95 51.25) (width 0.3) (layer "F.Cu") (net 4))
 (segment (start 28.5 52.45) (end 622.65 52.45) (width 0.5) (layer "F.Cu") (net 4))
 (via (at 622.2 51.25) (size 0.3) (drill 0.125) (layers "F.Cu" "B.Cu") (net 4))
 (via (at 28.85 51.25) (size 0.3) (drill 0.125) (layers "F.Cu" "B.Cu") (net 4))
 (via (at 27.95 51.25) (size 0.3) (drill 0.125) (layers "F.Cu" "B.Cu") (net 4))
 (via (at 28.5 52.45) (size 0.7) (drill 0.3) (layers "F.Cu" "B.Cu") (free) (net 4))
 (via (at 28.5 53.2) (size 0.7) (drill 0.3) (layers "F.Cu" "B.Cu") (free) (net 4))
 (via (at 28.4 51.25) (size 0.3) (drill 0.125) (layers "F.Cu" "B.Cu") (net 4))
 (via (at 28.6 48.5) (size 0.7) (drill 0.3) (layers "F.Cu" "B.Cu") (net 4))
 (segment (start 25.5 51.25) (end 25.598629 51.25) (width 0.5) (layer "B.Cu") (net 4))
 (segment (start 622.2 51.25) (end 622.85 51.25) (width 0.3) (layer "B.Cu") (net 4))
 (segment (start 623.77 48.75) (end 622.85 48.75) (width 0.3) (layer "B.Cu") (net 4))
 (segment (start 27.750001 50.25) (end 27.775001 50.225) (width 0.2) (layer "F.Cu") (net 6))
 (segment (start 27.15 50.25) (end 27.750001 50.25) (width 0.2) (layer "F.Cu") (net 6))
 (segment (start 27.775001 50.225) (end 621.550001 50.225001) (width 0.2) (layer "F.Cu") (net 6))
 (segment (start 621.550001 50.225001) (end 621.6 50.275) (width 0.2) (layer "F.Cu") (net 6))
 (via (at 621.6 50.275) (size 0.3) (drill 0.125) (layers "F.Cu" "B.Cu") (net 6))
 (segment (start 622.224999 50.225) (end 622.249999 50.25) (width 0.2) (layer "B.Cu") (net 6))
 (segment (start 621.65 50.225) (end 622.224999 50.225) (width 0.2) (layer "B.Cu") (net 6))
 (segment (start 621.6 50.275) (end 621.65 50.225) (width 0.2) (layer "B.Cu") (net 6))
 (segment (start 622.249999 50.25) (end 622.85 50.25) (width 0.2) (layer "B.Cu") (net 6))
 (segment (start 27.15 49.75) (end 27.750001 49.75) (width 0.2) (layer "F.Cu") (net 7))
 (segment (start 27.775001 49.775) (end 621.550001 49.774999) (width 0.2) (layer "F.Cu") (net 7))
 (segment (start 27.750001 49.75) (end 27.775001 49.775) (width 0.2) (layer "F.Cu") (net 7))
 (segment (start 621.550001 49.774999) (end 621.6 49.725) (width 0.2) (layer "F.Cu") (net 7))
 (via (at 621.6 49.725) (size 0.3) (drill 0.125) (layers "F.Cu" "B.Cu") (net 7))
 (segment (start 621.65 49.775) (end 622.224999 49.775) (width 0.2) (layer "B.Cu") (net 7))
 (segment (start 622.224999 49.775) (end 622.249999 49.75) (width 0.2) (layer "B.Cu") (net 7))
 (segment (start 622.249999 49.75) (end 622.85 49.75) (width 0.2) (layer "B.Cu") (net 7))
 (segment (start 621.6 49.725) (end 621.65 49.775) (width 0.2) (layer "B.Cu") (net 7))
 (segment (start 27.15 50.75) (end 620.95 50.75) (width 0.3) (layer "F.Cu") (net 5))
 (via (at 620.95 50.75) (size 0.3) (drill 0.125) (layers "F.Cu" "B.Cu") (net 5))
 (segment (start 621.25 50.9) (end 621.1 50.75) (width 0.3) (layer "B.Cu") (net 5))
 (segment (start 620.95 50.75) (end 621.1 50.75) (width 0.3) (layer "B.Cu") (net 5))
 (segment (start 622.85 50.75) (end 621.992893 50.75) (width 0.3) (layer "B.Cu") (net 5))
 (segment (start 621.842893 50.9) (end 621.25 50.9) (width 0.3) (layer "B.Cu") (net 5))
 (segment (start 621.992893 50.75) (end 621.842893 50.9) (width 0.3) (layer "B.Cu") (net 5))
 (segment (start 27.15 49.25) (end 620.95 49.25) (width 0.3) (layer "F.Cu") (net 8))
 (via (at 620.95 49.25) (size 0.3) (drill 0.125) (layers "F.Cu" "B.Cu") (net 8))
 (segment (start 621.827818 49.175) (end 621.372182 49.175) (width 0.3) (layer "B.Cu") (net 8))
 (segment (start 621.372182 49.175) (end 621.297182 49.25) (width 0.3) (layer "B.Cu") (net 8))
 (segment (start 621.297182 49.25) (end 620.95 49.25) (width 0.3) (layer "B.Cu") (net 8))
 (segment (start 622.85 49.25) (end 621.902818 49.25) (width 0.3) (layer "B.Cu") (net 8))
 (segment (start 621.902818 49.25) (end 621.827818 49.175) (width 0.3) (layer "B.Cu") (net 8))
 (segment (start 26.23 47.75) (end 27.15 47.75) (width 0.3) (layer "F.Cu") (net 10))
 (segment (start 27.15 47.75) (end 623.77 47.75) (width 0.3) (layer "F.Cu") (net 10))
 (segment (start 624 47.75) (end 624.5 48.25) (width 0.3) (layer "F.Cu") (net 10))
 (segment (start 25.73 48.25) (end 26.23 47.75) (width 0.3) (layer "F.Cu") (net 10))
 (segment (start 623.77 47.75) (end 624 47.75) (width 0.3) (layer "F.Cu") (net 10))
 (segment (start 624.5 48.25) (end 624.5 49.25) (width 0.3) (layer "F.Cu") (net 10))
 (segment (start 25.5 48.25) (end 25.73 48.25) (width 0.3) (layer "F.Cu") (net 10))
 (segment (start 25.5 49.25) (end 25.5 48.25) (width 0.3) (layer "F.Cu") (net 10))
 (segment (start 622.31703 51.75) (end 623.77 51.75) (width 0.3) (layer "F.Cu") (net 3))
 (segment (start 27.15 51.75) (end 620.882968 51.75) (width 0.3) (layer "F.Cu") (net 3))
 (segment (start 623.77 51.75) (end 623.77 50.75) (width 0.3) (layer "F.Cu") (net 3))
 (segment (start 622.242027 51.825002) (end 622.31703 51.75) (width 0.3) (layer "F.Cu") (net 3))
 (segment (start 26.23 51.75) (end 27.15 51.75) (width 0.3) (layer "F.Cu") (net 3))
 (segment (start 620.882968 51.75) (end 620.957968 51.825) (width 0.3) (layer "F.Cu") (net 3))
 (segment (start 26.23 50.75) (end 26.23 51.75) (width 0.3) (layer "F.Cu") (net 3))
 (segment (start 620.957968 51.825) (end 622.242027 51.825002) (width 0.3) (layer "F.Cu") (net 3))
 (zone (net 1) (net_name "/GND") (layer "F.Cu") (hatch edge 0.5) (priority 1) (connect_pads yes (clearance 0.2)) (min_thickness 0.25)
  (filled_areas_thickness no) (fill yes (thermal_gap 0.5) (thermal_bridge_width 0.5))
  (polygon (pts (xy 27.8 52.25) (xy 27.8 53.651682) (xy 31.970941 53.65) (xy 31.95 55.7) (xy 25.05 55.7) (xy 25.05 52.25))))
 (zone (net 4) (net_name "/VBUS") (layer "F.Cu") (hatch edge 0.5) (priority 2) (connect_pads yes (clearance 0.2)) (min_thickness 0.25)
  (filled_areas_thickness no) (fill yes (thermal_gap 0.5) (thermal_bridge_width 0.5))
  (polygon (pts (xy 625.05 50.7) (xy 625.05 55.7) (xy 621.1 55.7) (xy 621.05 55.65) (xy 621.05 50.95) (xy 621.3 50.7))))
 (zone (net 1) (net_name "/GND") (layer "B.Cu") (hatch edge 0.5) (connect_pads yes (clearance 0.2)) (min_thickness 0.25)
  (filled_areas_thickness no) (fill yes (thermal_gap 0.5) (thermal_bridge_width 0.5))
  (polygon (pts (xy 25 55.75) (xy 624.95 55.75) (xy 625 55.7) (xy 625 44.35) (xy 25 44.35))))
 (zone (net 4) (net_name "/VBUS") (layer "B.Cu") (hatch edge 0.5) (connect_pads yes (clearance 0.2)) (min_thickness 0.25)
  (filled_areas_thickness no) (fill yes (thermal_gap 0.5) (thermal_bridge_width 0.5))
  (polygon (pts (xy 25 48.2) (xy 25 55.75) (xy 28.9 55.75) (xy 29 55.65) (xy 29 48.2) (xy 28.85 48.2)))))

